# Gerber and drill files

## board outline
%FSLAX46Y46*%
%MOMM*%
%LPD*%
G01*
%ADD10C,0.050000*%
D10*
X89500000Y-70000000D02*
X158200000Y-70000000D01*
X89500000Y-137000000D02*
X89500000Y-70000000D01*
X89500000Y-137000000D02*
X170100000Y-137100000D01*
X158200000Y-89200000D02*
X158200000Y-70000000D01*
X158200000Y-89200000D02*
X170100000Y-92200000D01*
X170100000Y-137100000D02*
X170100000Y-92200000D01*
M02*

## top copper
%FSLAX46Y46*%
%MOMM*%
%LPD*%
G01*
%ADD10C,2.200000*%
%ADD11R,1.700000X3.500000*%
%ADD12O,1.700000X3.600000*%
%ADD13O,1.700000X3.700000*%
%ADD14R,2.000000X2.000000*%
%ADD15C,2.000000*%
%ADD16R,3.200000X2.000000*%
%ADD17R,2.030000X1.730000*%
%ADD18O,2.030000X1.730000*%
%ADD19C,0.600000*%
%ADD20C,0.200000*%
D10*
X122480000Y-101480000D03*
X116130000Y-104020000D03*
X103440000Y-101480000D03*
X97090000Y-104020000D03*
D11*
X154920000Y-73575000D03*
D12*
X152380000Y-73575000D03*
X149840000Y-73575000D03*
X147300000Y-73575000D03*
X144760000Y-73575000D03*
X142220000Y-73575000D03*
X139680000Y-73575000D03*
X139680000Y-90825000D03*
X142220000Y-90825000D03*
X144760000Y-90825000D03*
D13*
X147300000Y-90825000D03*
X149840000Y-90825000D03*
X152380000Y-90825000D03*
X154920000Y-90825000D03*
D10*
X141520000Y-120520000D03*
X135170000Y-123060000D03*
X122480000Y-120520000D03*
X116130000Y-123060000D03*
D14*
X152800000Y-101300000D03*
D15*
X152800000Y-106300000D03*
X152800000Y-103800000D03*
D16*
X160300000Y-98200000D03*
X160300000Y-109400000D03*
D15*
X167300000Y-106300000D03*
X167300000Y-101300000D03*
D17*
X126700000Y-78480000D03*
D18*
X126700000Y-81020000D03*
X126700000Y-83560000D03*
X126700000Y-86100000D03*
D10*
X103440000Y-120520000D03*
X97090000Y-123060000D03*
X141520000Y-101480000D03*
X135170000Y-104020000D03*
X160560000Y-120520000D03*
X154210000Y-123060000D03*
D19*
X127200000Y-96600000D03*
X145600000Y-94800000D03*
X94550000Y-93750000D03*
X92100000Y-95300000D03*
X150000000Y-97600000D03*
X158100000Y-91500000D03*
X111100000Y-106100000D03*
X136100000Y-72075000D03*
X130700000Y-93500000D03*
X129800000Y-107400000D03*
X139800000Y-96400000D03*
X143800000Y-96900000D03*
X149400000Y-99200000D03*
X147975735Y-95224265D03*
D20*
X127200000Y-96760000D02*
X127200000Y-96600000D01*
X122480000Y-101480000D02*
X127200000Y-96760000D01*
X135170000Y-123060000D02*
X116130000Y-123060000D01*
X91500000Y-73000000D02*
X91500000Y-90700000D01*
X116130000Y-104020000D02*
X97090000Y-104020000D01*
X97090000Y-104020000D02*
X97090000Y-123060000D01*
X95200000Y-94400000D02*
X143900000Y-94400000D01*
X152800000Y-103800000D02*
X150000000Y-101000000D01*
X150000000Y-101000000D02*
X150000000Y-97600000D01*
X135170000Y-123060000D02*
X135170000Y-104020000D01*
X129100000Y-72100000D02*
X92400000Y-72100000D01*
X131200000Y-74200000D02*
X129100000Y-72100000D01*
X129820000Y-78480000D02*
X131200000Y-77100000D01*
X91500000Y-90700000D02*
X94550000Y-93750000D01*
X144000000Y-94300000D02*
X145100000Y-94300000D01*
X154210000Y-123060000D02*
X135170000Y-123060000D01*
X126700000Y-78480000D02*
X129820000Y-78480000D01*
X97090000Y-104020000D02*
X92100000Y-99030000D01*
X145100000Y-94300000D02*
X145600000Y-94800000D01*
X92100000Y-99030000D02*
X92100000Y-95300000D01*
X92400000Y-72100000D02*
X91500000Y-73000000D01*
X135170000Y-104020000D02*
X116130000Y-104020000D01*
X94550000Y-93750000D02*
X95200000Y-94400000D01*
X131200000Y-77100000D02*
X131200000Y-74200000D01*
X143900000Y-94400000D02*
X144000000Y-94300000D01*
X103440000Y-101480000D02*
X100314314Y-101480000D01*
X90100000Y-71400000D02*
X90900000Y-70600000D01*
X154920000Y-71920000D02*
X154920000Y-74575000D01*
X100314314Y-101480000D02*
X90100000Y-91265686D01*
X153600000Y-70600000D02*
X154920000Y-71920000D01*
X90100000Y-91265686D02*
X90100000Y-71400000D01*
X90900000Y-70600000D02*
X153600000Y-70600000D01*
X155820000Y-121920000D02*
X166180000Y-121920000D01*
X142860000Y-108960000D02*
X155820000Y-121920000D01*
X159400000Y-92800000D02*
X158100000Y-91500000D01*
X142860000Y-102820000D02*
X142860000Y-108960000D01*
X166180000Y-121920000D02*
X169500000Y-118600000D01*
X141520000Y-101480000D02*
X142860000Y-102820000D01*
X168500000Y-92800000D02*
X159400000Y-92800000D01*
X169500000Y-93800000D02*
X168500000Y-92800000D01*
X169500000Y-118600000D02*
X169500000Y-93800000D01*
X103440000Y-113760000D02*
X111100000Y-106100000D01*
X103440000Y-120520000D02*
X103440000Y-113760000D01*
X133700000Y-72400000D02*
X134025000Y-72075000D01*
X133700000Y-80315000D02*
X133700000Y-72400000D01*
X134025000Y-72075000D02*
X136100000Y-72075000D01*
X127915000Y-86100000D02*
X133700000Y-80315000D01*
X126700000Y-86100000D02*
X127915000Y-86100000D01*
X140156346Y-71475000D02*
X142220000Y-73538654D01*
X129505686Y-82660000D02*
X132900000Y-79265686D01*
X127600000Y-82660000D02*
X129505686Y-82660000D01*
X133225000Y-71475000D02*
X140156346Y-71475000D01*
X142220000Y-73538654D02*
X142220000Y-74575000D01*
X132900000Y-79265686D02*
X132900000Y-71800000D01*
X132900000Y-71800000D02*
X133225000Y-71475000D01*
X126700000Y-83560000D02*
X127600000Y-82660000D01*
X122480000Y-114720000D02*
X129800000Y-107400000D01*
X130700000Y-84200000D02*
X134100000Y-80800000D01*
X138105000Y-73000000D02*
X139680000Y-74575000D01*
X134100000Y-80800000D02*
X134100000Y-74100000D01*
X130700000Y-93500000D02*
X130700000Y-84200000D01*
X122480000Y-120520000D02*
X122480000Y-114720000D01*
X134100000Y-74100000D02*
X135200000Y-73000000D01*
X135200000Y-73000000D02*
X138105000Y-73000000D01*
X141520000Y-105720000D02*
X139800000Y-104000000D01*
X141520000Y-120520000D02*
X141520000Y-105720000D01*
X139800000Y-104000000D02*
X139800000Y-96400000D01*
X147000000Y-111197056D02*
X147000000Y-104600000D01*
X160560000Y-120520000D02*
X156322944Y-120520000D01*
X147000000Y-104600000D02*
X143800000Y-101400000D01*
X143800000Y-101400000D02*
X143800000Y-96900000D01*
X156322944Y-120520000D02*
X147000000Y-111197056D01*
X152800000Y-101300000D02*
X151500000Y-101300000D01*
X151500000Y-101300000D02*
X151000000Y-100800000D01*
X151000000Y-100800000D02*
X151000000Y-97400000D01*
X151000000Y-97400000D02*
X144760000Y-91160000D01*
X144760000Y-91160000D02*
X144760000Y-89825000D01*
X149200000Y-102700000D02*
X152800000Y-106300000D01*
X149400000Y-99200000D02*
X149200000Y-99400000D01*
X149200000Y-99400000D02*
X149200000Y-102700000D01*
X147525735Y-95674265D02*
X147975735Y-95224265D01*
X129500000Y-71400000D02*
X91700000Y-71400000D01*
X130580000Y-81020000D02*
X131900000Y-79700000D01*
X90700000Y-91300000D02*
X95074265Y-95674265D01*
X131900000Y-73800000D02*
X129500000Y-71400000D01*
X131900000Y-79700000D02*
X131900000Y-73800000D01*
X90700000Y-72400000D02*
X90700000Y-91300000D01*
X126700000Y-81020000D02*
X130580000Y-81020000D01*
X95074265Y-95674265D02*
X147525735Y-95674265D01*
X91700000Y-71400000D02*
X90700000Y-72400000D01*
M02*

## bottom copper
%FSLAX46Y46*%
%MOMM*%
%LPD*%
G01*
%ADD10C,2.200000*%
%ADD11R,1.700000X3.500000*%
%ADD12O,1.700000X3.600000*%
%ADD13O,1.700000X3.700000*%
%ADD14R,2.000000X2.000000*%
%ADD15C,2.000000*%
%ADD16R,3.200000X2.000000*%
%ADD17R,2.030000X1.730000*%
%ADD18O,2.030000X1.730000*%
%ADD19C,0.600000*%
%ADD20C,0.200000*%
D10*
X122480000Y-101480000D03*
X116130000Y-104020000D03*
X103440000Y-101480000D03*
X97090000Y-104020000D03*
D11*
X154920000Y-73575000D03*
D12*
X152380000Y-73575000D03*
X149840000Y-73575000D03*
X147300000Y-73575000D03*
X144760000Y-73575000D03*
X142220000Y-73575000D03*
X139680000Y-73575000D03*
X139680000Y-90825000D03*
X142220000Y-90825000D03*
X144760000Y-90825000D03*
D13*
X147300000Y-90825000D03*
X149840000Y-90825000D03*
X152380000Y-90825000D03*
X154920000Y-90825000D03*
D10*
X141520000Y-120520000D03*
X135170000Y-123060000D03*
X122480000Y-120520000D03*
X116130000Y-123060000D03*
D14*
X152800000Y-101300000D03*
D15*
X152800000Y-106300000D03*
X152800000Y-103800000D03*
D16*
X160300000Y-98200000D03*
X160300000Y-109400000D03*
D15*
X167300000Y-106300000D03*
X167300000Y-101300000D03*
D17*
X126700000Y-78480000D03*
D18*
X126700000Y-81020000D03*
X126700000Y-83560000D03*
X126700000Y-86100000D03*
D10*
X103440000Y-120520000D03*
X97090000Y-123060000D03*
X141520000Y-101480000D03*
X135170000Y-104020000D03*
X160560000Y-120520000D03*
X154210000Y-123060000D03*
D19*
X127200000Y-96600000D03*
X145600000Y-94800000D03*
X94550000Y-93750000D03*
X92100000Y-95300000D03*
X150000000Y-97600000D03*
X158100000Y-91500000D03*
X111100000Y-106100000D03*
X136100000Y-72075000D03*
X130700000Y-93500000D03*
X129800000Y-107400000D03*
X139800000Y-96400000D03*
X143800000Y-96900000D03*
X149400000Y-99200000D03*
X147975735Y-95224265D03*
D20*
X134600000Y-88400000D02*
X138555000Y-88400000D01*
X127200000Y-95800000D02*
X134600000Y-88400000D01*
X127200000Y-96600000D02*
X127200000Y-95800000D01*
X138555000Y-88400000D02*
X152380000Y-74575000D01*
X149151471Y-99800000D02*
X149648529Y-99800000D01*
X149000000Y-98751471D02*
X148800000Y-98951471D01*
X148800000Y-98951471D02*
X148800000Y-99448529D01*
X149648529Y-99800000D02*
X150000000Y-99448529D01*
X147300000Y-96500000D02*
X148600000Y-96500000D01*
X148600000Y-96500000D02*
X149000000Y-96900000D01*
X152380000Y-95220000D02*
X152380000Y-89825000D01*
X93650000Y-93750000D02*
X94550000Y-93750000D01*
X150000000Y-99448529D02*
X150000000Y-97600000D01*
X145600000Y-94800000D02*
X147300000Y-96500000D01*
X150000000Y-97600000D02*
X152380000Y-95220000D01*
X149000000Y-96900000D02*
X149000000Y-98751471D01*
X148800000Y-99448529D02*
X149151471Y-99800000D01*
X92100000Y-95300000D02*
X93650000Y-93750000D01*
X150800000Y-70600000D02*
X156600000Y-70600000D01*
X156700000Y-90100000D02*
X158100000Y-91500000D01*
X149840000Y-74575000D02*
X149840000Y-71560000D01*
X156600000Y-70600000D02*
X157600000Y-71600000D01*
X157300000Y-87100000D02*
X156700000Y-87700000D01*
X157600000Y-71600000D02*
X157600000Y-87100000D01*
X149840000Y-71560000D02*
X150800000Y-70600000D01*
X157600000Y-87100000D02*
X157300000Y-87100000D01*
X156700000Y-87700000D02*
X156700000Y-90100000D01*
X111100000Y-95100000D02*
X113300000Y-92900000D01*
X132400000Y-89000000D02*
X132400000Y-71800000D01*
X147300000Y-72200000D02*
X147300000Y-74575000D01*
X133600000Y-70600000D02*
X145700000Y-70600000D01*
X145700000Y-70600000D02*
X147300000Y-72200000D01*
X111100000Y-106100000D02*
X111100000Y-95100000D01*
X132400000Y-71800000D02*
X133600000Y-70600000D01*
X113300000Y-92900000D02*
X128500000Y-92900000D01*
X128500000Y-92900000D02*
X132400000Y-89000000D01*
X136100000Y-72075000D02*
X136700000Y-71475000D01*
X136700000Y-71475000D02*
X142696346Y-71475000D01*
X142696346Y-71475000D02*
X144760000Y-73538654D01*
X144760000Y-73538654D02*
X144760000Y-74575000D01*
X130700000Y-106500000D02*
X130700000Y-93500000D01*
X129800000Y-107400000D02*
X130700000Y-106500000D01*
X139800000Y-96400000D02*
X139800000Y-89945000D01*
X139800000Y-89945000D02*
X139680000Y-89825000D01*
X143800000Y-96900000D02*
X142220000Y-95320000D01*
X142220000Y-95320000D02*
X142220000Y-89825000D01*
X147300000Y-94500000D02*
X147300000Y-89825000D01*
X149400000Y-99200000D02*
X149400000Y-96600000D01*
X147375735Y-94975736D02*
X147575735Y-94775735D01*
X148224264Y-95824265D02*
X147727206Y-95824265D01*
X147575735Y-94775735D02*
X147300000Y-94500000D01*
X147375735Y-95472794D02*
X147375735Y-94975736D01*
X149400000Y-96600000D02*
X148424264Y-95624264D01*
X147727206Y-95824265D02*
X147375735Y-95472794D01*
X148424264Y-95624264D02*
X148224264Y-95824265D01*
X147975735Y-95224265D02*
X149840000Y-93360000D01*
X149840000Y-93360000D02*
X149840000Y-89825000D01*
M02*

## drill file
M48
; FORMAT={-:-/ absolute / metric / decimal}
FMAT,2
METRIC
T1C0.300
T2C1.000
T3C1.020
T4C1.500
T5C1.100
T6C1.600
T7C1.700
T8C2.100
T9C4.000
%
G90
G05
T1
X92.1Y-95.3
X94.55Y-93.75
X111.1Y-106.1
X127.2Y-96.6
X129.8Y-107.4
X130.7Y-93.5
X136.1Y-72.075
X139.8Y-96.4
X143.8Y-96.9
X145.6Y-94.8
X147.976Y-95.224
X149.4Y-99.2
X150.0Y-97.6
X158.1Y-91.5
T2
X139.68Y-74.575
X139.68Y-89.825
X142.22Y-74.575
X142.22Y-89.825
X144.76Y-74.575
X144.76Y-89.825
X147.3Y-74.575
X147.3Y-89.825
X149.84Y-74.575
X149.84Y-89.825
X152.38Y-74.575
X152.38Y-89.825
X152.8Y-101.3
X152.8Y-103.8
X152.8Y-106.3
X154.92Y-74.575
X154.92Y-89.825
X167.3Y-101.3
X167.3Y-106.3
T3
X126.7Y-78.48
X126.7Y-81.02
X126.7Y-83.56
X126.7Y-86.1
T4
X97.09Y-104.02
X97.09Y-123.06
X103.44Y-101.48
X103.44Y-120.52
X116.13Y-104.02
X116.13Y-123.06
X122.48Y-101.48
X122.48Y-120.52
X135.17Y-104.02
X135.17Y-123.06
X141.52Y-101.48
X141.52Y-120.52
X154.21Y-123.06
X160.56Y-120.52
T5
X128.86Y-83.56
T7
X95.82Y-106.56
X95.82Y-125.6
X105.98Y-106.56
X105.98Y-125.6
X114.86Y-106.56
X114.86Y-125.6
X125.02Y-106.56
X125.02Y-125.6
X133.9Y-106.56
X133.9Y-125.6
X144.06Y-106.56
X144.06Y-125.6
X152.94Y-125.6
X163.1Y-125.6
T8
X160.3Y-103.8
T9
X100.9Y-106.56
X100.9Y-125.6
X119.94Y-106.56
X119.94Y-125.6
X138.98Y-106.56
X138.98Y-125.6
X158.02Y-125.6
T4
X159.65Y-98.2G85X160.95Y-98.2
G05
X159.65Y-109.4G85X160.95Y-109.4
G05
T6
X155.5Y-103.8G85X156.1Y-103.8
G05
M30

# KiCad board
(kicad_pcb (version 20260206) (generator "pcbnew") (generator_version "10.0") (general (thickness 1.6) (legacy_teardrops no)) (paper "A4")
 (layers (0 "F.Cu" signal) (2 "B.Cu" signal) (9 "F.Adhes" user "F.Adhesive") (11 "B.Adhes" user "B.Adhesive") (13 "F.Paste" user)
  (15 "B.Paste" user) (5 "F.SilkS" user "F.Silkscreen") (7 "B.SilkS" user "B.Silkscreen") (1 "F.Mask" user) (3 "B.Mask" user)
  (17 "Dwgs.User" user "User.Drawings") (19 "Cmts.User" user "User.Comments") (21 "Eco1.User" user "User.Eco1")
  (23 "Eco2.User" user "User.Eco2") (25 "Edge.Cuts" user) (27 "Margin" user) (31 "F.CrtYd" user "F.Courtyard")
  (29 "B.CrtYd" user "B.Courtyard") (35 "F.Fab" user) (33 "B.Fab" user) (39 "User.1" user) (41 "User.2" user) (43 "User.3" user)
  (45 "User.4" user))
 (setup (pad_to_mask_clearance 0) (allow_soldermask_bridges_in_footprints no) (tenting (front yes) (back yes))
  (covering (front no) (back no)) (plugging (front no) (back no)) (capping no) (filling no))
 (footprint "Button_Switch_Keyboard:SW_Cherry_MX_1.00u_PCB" (layer "F.Cu") (at 122.48 101.48)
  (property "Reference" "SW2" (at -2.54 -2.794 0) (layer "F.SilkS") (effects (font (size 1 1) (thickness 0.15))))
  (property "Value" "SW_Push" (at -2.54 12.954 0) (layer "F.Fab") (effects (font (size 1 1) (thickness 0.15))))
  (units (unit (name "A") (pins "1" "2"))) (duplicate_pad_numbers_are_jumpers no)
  (pad "" np_thru_hole circle (at -7.62 5.08) (size 1.7 1.7) (drill 1.7) (layers "*.Cu" "*.Mask"))
  (pad "" np_thru_hole circle (at -2.54 5.08) (size 4 4) (drill 4) (layers "*.Cu" "*.Mask"))
  (pad "" np_thru_hole circle (at 2.54 5.08) (size 1.7 1.7) (drill 1.7) (layers "*.Cu" "*.Mask"))
  (pad "1" thru_hole circle (at 0 0) (size 2.2 2.2) (drill 1.5) (layers "*.Cu" "*.Mask") (remove_unused_layers no) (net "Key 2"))
  (pad "2" thru_hole circle (at -6.35 2.54) (size 2.2 2.2) (drill 1.5) (layers "*.Cu" "*.Mask") (remove_unused_layers no) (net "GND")))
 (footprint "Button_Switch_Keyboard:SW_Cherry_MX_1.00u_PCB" (layer "F.Cu") (at 103.44 101.48)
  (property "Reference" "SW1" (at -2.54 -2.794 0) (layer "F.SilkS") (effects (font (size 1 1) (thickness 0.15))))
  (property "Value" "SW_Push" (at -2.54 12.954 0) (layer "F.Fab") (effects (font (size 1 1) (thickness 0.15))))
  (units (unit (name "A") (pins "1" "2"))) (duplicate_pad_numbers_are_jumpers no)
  (pad "" np_thru_hole circle (at -7.62 5.08) (size 1.7 1.7) (drill 1.7) (layers "*.Cu" "*.Mask"))
  (pad "" np_thru_hole circle (at -2.54 5.08) (size 4 4) (drill 4) (layers "*.Cu" "*.Mask"))
  (pad "" np_thru_hole circle (at 2.54 5.08) (size 1.7 1.7) (drill 1.7) (layers "*.Cu" "*.Mask"))
  (pad "1" thru_hole circle (at 0 0) (size 2.2 2.2) (drill 1.5) (layers "*.Cu" "*.Mask") (remove_unused_layers no) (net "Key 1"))
  (pad "2" thru_hole circle (at -6.35 2.54) (size 2.2 2.2) (drill 1.5) (layers "*.Cu" "*.Mask") (remove_unused_layers no) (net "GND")))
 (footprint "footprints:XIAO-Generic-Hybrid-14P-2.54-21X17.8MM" (layer "F.Cu") (at 147.3 82.2 -90)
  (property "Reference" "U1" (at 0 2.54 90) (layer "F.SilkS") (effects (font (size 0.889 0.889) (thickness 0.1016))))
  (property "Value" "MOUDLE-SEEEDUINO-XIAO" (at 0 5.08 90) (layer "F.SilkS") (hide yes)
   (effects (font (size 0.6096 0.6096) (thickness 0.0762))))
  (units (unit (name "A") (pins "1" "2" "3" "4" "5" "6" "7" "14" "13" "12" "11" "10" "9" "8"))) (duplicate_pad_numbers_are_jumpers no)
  (pad "1" thru_hole rect (at -7.625 -7.62 270) (size 3.5 1.7) (drill 1 (offset -1 0)) (layers "*.Cu" "*.Mask") (remove_unused_layers no)
   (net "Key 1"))
  (pad "2" thru_hole oval (at -7.625 -5.08 270) (size 3.6 1.7) (drill 1 (offset -1 0)) (layers "*.Cu" "*.Mask") (remove_unused_layers no)
   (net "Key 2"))
  (pad "3" thru_hole oval (at -7.625 -2.54 270) (size 3.6 1.7) (drill 1 (offset -1 0)) (layers "*.Cu" "*.Mask") (remove_unused_layers no)
   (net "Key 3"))
  (pad "4" thru_hole oval (at -7.625 0 270) (size 3.6 1.7) (drill 1 (offset -1 0)) (layers "*.Cu" "*.Mask") (remove_unused_layers no)
   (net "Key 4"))
  (pad "5" thru_hole oval (at -7.625 2.54 270) (size 3.6 1.7) (drill 1 (offset -1 0)) (layers "*.Cu" "*.Mask") (remove_unused_layers no)
   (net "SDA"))
  (pad "6" thru_hole oval (at -7.625 5.08 90) (size 3.6 1.7) (drill 1 (offset 1 0)) (layers "*.Cu" "*.Mask") (remove_unused_layers no)
   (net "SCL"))
  (pad "7" thru_hole oval (at -7.625 7.62 270) (size 3.6 1.7) (drill 1 (offset -1 0)) (layers "*.Cu" "*.Mask") (remove_unused_layers no)
   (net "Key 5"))
  (pad "8" thru_hole oval (at 7.625 7.62 270) (size 3.6 1.7) (drill 1 (offset 1 0)) (layers "*.Cu" "*.Mask") (remove_unused_layers no)
   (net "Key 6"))
  (pad "9" thru_hole oval (at 7.625 5.08 270) (size 3.6 1.7) (drill 1 (offset 1 0)) (layers "*.Cu" "*.Mask") (remove_unused_layers no)
   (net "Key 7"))
  (pad "10" thru_hole oval (at 7.625 2.54 270) (size 3.6 1.7) (drill 1 (offset 1 0)) (layers "*.Cu" "*.Mask") (remove_unused_layers no)
   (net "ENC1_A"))
  (pad "11" thru_hole oval (at 7.625 0 270) (size 3.7 1.7) (drill 1 (offset 1 0)) (layers "*.Cu" "*.Mask") (remove_unused_layers no)
   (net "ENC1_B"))
  (pad "12" thru_hole oval (at 7.625 -2.54 270) (size 3.7 1.7) (drill 1 (offset 1 0)) (layers "*.Cu" "*.Mask") (remove_unused_layers no)
   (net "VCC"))
  (pad "13" thru_hole oval (at 7.625 -5.08 270) (size 3.7 1.7) (drill 1 (offset 1 0)) (layers "*.Cu" "*.Mask") (remove_unused_layers no)
   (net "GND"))
  (pad "14" thru_hole oval (at 7.625 -7.62 270) (size 3.7 1.7) (drill 1 (offset 1 0)) (layers "*.Cu" "*.Mask") (remove_unused_layers no)
   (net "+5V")))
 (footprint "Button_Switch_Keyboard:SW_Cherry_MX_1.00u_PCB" (layer "F.Cu") (at 141.52 120.52)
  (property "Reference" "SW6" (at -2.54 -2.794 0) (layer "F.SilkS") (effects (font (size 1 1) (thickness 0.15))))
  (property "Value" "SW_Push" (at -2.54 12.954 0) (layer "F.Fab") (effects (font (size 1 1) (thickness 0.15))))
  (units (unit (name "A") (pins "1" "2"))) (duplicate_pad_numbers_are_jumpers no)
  (pad "" np_thru_hole circle (at -7.62 5.08) (size 1.7 1.7) (drill 1.7) (layers "*.Cu" "*.Mask"))
  (pad "" np_thru_hole circle (at -2.54 5.08) (size 4 4) (drill 4) (layers "*.Cu" "*.Mask"))
  (pad "" np_thru_hole circle (at 2.54 5.08) (size 1.7 1.7) (drill 1.7) (layers "*.Cu" "*.Mask"))
  (pad "1" thru_hole circle (at 0 0) (size 2.2 2.2) (drill 1.5) (layers "*.Cu" "*.Mask") (remove_unused_layers no) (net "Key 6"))
  (pad "2" thru_hole circle (at -6.35 2.54) (size 2.2 2.2) (drill 1.5) (layers "*.Cu" "*.Mask") (remove_unused_layers no) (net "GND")))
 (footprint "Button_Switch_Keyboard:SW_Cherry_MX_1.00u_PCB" (layer "F.Cu") (at 122.48 120.52)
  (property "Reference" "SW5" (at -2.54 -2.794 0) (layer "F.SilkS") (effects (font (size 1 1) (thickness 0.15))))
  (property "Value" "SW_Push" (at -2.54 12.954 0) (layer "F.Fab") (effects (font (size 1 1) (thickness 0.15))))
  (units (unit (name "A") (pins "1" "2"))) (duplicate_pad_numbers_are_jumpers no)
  (pad "" np_thru_hole circle (at -7.62 5.08) (size 1.7 1.7) (drill 1.7) (layers "*.Cu" "*.Mask"))
  (pad "" np_thru_hole circle (at -2.54 5.08) (size 4 4) (drill 4) (layers "*.Cu" "*.Mask"))
  (pad "" np_thru_hole circle (at 2.54 5.08) (size 1.7 1.7) (drill 1.7) (layers "*.Cu" "*.Mask"))
  (pad "1" thru_hole circle (at 0 0) (size 2.2 2.2) (drill 1.5) (layers "*.Cu" "*.Mask") (remove_unused_layers no) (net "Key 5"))
  (pad "2" thru_hole circle (at -6.35 2.54) (size 2.2 2.2) (drill 1.5) (layers "*.Cu" "*.Mask") (remove_unused_layers no) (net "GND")))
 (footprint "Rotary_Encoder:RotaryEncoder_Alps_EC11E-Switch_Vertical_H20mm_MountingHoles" (layer "F.Cu") (at 152.8 101.3)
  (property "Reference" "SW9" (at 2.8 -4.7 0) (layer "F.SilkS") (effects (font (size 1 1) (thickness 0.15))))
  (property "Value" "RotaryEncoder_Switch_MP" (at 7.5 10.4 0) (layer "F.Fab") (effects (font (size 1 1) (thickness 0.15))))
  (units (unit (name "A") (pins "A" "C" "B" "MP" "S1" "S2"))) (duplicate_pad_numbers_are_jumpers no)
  (pad "" np_thru_hole oval (at 3 2.5) (size 2.2 1.6) (drill oval 2.2 1.6) (layers "*.Mask"))
  (pad "" np_thru_hole circle (at 7.5 2.5) (size 2.1 2.1) (drill 2.1) (layers "*.Mask"))
  (pad "A" thru_hole rect (at 0 0) (size 2 2) (drill 1) (layers "*.Cu" "*.Mask") (remove_unused_layers no) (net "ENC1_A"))
  (pad "B" thru_hole circle (at 0 5) (size 2 2) (drill 1) (layers "*.Cu" "*.Mask") (remove_unused_layers no) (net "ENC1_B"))
  (pad "C" thru_hole circle (at 0 2.5) (size 2 2) (drill 1) (layers "*.Cu" "*.Mask") (remove_unused_layers no) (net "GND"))
  (pad "MP" thru_hole rect (at 7.5 -3.1) (size 3.2 2) (drill oval 2.8 1.5) (layers "*.Cu" "*.Mask") (remove_unused_layers no)
   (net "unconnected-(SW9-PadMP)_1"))
  (pad "MP" thru_hole rect (at 7.5 8.1) (size 3.2 2) (drill oval 2.8 1.5) (layers "*.Cu" "*.Mask") (remove_unused_layers no)
   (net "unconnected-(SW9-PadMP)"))
  (pad "S1" thru_hole circle (at 14.5 5) (size 2 2) (drill 1) (layers "*.Cu" "*.Mask") (remove_unused_layers no)
   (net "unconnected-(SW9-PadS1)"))
  (pad "S2" thru_hole circle (at 14.5 0) (size 2 2) (drill 1) (layers "*.Cu" "*.Mask") (remove_unused_layers no)
   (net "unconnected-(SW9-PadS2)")))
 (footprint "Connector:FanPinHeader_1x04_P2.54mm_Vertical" (layer "F.Cu") (at 126.7 78.48 -90)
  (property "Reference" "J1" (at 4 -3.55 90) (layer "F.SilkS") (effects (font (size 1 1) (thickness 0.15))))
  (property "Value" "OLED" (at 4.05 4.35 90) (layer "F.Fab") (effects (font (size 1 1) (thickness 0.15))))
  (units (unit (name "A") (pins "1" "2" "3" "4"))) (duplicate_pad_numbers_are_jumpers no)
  (pad "" np_thru_hole circle (at 5.08 -2.16) (size 1.1 1.1) (drill 1.1) (layers "*.Cu" "*.Mask"))
  (pad "1" thru_hole rect (at 0 0) (size 2.03 1.73) (drill 1.02) (layers "*.Cu" "*.Mask") (remove_unused_layers no) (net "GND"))
  (pad "2" thru_hole oval (at 2.54 0) (size 2.03 1.73) (drill 1.02) (layers "*.Cu" "*.Mask") (remove_unused_layers no) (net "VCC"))
  (pad "3" thru_hole oval (at 5.08 0) (size 2.03 1.73) (drill 1.02) (layers "*.Cu" "*.Mask") (remove_unused_layers no) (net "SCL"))
  (pad "4" thru_hole oval (at 7.62 0) (size 2.03 1.73) (drill 1.02) (layers "*.Cu" "*.Mask") (remove_unused_layers no) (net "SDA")))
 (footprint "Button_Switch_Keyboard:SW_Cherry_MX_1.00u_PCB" (layer "F.Cu") (at 103.44 120.52)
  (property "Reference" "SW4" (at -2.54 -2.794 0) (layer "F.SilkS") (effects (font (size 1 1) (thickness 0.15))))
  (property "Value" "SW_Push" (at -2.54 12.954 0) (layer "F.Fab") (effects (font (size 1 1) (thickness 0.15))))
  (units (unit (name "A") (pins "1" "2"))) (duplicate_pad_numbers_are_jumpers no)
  (pad "" np_thru_hole circle (at -7.62 5.08) (size 1.7 1.7) (drill 1.7) (layers "*.Cu" "*.Mask"))
  (pad "" np_thru_hole circle (at -2.54 5.08) (size 4 4) (drill 4) (layers "*.Cu" "*.Mask"))
  (pad "" np_thru_hole circle (at 2.54 5.08) (size 1.7 1.7) (drill 1.7) (layers "*.Cu" "*.Mask"))
  (pad "1" thru_hole circle (at 0 0) (size 2.2 2.2) (drill 1.5) (layers "*.Cu" "*.Mask") (remove_unused_layers no) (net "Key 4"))
  (pad "2" thru_hole circle (at -6.35 2.54) (size 2.2 2.2) (drill 1.5) (layers "*.Cu" "*.Mask") (remove_unused_layers no) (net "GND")))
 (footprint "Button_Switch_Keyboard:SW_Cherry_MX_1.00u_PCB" (layer "F.Cu") (at 141.52 101.48)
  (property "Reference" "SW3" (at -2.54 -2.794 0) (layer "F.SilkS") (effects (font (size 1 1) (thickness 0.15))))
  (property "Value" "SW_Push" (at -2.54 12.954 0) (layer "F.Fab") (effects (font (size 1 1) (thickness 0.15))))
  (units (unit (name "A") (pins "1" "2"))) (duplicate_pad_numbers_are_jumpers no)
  (pad "" np_thru_hole circle (at -7.62 5.08) (size 1.7 1.7) (drill 1.7) (layers "*.Cu" "*.Mask"))
  (pad "" np_thru_hole circle (at -2.54 5.08) (size 4 4) (drill 4) (layers "*.Cu" "*.Mask"))
  (pad "" np_thru_hole circle (at 2.54 5.08) (size 1.7 1.7) (drill 1.7) (layers "*.Cu" "*.Mask"))
  (pad "1" thru_hole circle (at 0 0) (size 2.2 2.2) (drill 1.5) (layers "*.Cu" "*.Mask") (remove_unused_layers no) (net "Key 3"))
  (pad "2" thru_hole circle (at -6.35 2.54) (size 2.2 2.2) (drill 1.5) (layers "*.Cu" "*.Mask") (remove_unused_layers no) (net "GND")))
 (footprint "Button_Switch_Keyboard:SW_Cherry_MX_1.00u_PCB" (layer "F.Cu") (at 160.56 120.52)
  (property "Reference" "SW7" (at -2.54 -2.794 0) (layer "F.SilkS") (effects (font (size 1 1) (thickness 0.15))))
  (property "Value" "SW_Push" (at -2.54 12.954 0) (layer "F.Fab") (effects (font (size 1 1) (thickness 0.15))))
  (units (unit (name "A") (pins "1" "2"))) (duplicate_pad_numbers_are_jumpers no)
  (pad "" np_thru_hole circle (at -7.62 5.08) (size 1.7 1.7) (drill 1.7) (layers "*.Cu" "*.Mask"))
  (pad "" np_thru_hole circle (at -2.54 5.08) (size 4 4) (drill 4) (layers "*.Cu" "*.Mask"))
  (pad "" np_thru_hole circle (at 2.54 5.08) (size 1.7 1.7) (drill 1.7) (layers "*.Cu" "*.Mask"))
  (pad "1" thru_hole circle (at 0 0) (size 2.2 2.2) (drill 1.5) (layers "*.Cu" "*.Mask") (remove_unused_layers no) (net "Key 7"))
  (pad "2" thru_hole circle (at -6.35 2.54) (size 2.2 2.2) (drill 1.5) (layers "*.Cu" "*.Mask") (remove_unused_layers no) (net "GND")))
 (gr_line (start 89.5 70) (end 158.2 70) (stroke (width 0.05) (type default)) (layer "Edge.Cuts"))
 (gr_line (start 89.5 137) (end 89.5 70) (stroke (width 0.05) (type default)) (layer "Edge.Cuts"))
 (gr_line (start 89.5 137) (end 170.1 137.1) (stroke (width 0.05) (type default)) (layer "Edge.Cuts"))
 (gr_line (start 158.2 89.2) (end 158.2 70) (stroke (width 0.05) (type default)) (layer "Edge.Cuts"))
 (gr_line (start 158.2 89.2) (end 170.1 92.2) (stroke (width 0.05) (type default)) (layer "Edge.Cuts"))
 (gr_line (start 170.1 137.1) (end 170.1 92.2) (stroke (width 0.05) (type default)) (layer "Edge.Cuts"))
 (segment (start 127.2 96.76) (end 127.2 96.6) (width 0.2) (layer "F.Cu") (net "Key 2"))
 (segment (start 122.48 101.48) (end 127.2 96.76) (width 0.2) (layer "F.Cu") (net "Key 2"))
 (via (at 127.2 96.6) (size 0.6) (drill 0.3) (layers "F.Cu" "B.Cu") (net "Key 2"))
 (segment (start 134.6 88.4) (end 138.555 88.4) (width 0.2) (layer "B.Cu") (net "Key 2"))
 (segment (start 127.2 95.8) (end 134.6 88.4) (width 0.2) (layer "B.Cu") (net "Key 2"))
 (segment (start 127.2 96.6) (end 127.2 95.8) (width 0.2) (layer "B.Cu") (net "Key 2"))
 (segment (start 138.555 88.4) (end 152.38 74.575) (width 0.2) (layer "B.Cu") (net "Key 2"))
 (segment (start 135.17 123.06) (end 116.13 123.06) (width 0.2) (layer "F.Cu") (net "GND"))
 (segment (start 91.5 73) (end 91.5 90.7) (width 0.2) (layer "F.Cu") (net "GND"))
 (segment (start 116.13 104.02) (end 97.09 104.02) (width 0.2) (layer "F.Cu") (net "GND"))
 (segment (start 97.09 104.02) (end 97.09 123.06) (width 0.2) (layer "F.Cu") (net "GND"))
 (segment (start 95.2 94.4) (end 143.9 94.4) (width 0.2) (layer "F.Cu") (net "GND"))
 (segment (start 152.8 103.8) (end 150 101) (width 0.2) (layer "F.Cu") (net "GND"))
 (segment (start 150 101) (end 150 97.6) (width 0.2) (layer "F.Cu") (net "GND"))
 (segment (start 135.17 123.06) (end 135.17 104.02) (width 0.2) (layer "F.Cu") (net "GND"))
 (segment (start 129.1 72.1) (end 92.4 72.1) (width 0.2) (layer "F.Cu") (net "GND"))
 (segment (start 131.2 74.2) (end 129.1 72.1) (width 0.2) (layer "F.Cu") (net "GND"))
 (segment (start 129.82 78.48) (end 131.2 77.1) (width 0.2) (layer "F.Cu") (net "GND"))
 (segment (start 91.5 90.7) (end 94.55 93.75) (width 0.2) (layer "F.Cu") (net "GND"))
 (segment (start 144 94.3) (end 145.1 94.3) (width 0.2) (layer "F.Cu") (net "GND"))
 (segment (start 154.21 123.06) (end 135.17 123.06) (width 0.2) (layer "F.Cu") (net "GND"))
 (segment (start 126.7 78.48) (end 129.82 78.48) (width 0.2) (layer "F.Cu") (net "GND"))
 (segment (start 97.09 104.02) (end 92.1 99.03) (width 0.2) (layer "F.Cu") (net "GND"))
 (segment (start 145.1 94.3) (end 145.6 94.8) (width 0.2) (layer "F.Cu") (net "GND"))
 (segment (start 92.1 99.03) (end 92.1 95.3) (width 0.2) (layer "F.Cu") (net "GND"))
 (segment (start 92.4 72.1) (end 91.5 73) (width 0.2) (layer "F.Cu") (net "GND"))
 (segment (start 135.17 104.02) (end 116.13 104.02) (width 0.2) (layer "F.Cu") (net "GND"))
 (segment (start 94.55 93.75) (end 95.2 94.4) (width 0.2) (layer "F.Cu") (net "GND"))
 (segment (start 131.2 77.1) (end 131.2 74.2) (width 0.2) (layer "F.Cu") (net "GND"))
 (segment (start 143.9 94.4) (end 144 94.3) (width 0.2) (layer "F.Cu") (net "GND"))
 (via (at 145.6 94.8) (size 0.6) (drill 0.3) (layers "F.Cu" "B.Cu") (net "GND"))
 (via (at 94.55 93.75) (size 0.6) (drill 0.3) (layers "F.Cu" "B.Cu") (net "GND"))
 (via (at 92.1 95.3) (size 0.6) (drill 0.3) (layers "F.Cu" "B.Cu") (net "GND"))
 (via (at 150 97.6) (size 0.6) (drill 0.3) (layers "F.Cu" "B.Cu") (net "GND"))
 (segment (start 149.151471 99.8) (end 149.648529 99.8) (width 0.2) (layer "B.Cu") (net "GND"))
 (segment (start 149 98.751471) (end 148.8 98.951471) (width 0.2) (layer "B.Cu") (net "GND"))
 (segment (start 148.8 98.951471) (end 148.8 99.448529) (width 0.2) (layer "B.Cu") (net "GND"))
 (segment (start 149.648529 99.8) (end 150 99.448529) (width 0.2) (layer "B.Cu") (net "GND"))
 (segment (start 147.3 96.5) (end 148.6 96.5) (width 0.2) (layer "B.Cu") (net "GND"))
 (segment (start 148.6 96.5) (end 149 96.9) (width 0.2) (layer "B.Cu") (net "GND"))
 (segment (start 152.38 95.22) (end 152.38 89.825) (width 0.2) (layer "B.Cu") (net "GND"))
 (segment (start 93.65 93.75) (end 94.55 93.75) (width 0.2) (layer "B.Cu") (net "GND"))
 (segment (start 150 99.448529) (end 150 97.6) (width 0.2) (layer "B.Cu") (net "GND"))
 (segment (start 145.6 94.8) (end 147.3 96.5) (width 0.2) (layer "B.Cu") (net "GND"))
 (segment (start 150 97.6) (end 152.38 95.22) (width 0.2) (layer "B.Cu") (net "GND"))
 (segment (start 149 96.9) (end 149 98.751471) (width 0.2) (layer "B.Cu") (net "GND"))
 (segment (start 148.8 99.448529) (end 149.151471 99.8) (width 0.2) (layer "B.Cu") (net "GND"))
 (segment (start 92.1 95.3) (end 93.65 93.75) (width 0.2) (layer "B.Cu") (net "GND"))
 (segment (start 103.44 101.48) (end 100.314314 101.48) (width 0.2) (layer "F.Cu") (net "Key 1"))
 (segment (start 90.1 71.4) (end 90.9 70.6) (width 0.2) (layer "F.Cu") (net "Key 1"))
 (segment (start 154.92 71.92) (end 154.92 74.575) (width 0.2) (layer "F.Cu") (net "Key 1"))
 (segment (start 100.314314 101.48) (end 90.1 91.265686) (width 0.2) (layer "F.Cu") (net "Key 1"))
 (segment (start 153.6 70.6) (end 154.92 71.92) (width 0.2) (layer "F.Cu") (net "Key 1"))
 (segment (start 90.1 91.265686) (end 90.1 71.4) (width 0.2) (layer "F.Cu") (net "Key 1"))
 (segment (start 90.9 70.6) (end 153.6 70.6) (width 0.2) (layer "F.Cu") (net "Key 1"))
 (segment (start 155.82 121.92) (end 166.18 121.92) (width 0.2) (layer "F.Cu") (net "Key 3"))
 (segment (start 142.86 108.96) (end 155.82 121.92) (width 0.2) (layer "F.Cu") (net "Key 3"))
 (segment (start 159.4 92.8) (end 158.1 91.5) (width 0.2) (layer "F.Cu") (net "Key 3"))
 (segment (start 142.86 102.82) (end 142.86 108.96) (width 0.2) (layer "F.Cu") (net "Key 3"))
 (segment (start 166.18 121.92) (end 169.5 118.6) (width 0.2) (layer "F.Cu") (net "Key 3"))
 (segment (start 141.52 101.48) (end 142.86 102.82) (width 0.2) (layer "F.Cu") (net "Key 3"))
 (segment (start 168.5 92.8) (end 159.4 92.8) (width 0.2) (layer "F.Cu") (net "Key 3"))
 (segment (start 169.5 93.8) (end 168.5 92.8) (width 0.2) (layer "F.Cu") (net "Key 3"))
 (segment (start 169.5 118.6) (end 169.5 93.8) (width 0.2) (layer "F.Cu") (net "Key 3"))
 (via (at 158.1 91.5) (size 0.6) (drill 0.3) (layers "F.Cu" "B.Cu") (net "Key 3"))
 (segment (start 150.8 70.6) (end 156.6 70.6) (width 0.2) (layer "B.Cu") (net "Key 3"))
 (segment (start 156.7 90.1) (end 158.1 91.5) (width 0.2) (layer "B.Cu") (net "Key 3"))
 (segment (start 149.84 74.575) (end 149.84 71.56) (width 0.2) (layer "B.Cu") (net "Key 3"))
 (segment (start 156.6 70.6) (end 157.6 71.6) (width 0.2) (layer "B.Cu") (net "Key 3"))
 (segment (start 157.3 87.1) (end 156.7 87.7) (width 0.2) (layer "B.Cu") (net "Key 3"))
 (segment (start 157.6 71.6) (end 157.6 87.1) (width 0.2) (layer "B.Cu") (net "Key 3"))
 (segment (start 149.84 71.56) (end 150.8 70.6) (width 0.2) (layer "B.Cu") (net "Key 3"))
 (segment (start 157.6 87.1) (end 157.3 87.1) (width 0.2) (layer "B.Cu") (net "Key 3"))
 (segment (start 156.7 87.7) (end 156.7 90.1) (width 0.2) (layer "B.Cu") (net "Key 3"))
 (segment (start 103.44 113.76) (end 111.1 106.1) (width 0.2) (layer "F.Cu") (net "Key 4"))
 (segment (start 103.44 120.52) (end 103.44 113.76) (width 0.2) (layer "F.Cu") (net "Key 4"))
 (via (at 111.1 106.1) (size 0.6) (drill 0.3) (layers "F.Cu" "B.Cu") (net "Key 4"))
 (segment (start 111.1 95.1) (end 113.3 92.9) (width 0.2) (layer "B.Cu") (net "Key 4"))
 (segment (start 132.4 89) (end 132.4 71.8) (width 0.2) (layer "B.Cu") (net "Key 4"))
 (segment (start 147.3 72.2) (end 147.3 74.575) (width 0.2) (layer "B.Cu") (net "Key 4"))
 (segment (start 133.6 70.6) (end 145.7 70.6) (width 0.2) (layer "B.Cu") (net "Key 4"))
 (segment (start 145.7 70.6) (end 147.3 72.2) (width 0.2) (layer "B.Cu") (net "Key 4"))
 (segment (start 111.1 106.1) (end 111.1 95.1) (width 0.2) (layer "B.Cu") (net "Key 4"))
 (segment (start 132.4 71.8) (end 133.6 70.6) (width 0.2) (layer "B.Cu") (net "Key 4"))
 (segment (start 113.3 92.9) (end 128.5 92.9) (width 0.2) (layer "B.Cu") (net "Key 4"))
 (segment (start 128.5 92.9) (end 132.4 89) (width 0.2) (layer "B.Cu") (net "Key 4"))
 (segment (start 133.7 72.4) (end 134.025 72.075) (width 0.2) (layer "F.Cu") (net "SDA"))
 (segment (start 133.7 80.315) (end 133.7 72.4) (width 0.2) (layer "F.Cu") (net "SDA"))
 (segment (start 134.025 72.075) (end 136.1 72.075) (width 0.2) (layer "F.Cu") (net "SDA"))
 (segment (start 127.915 86.1) (end 133.7 80.315) (width 0.2) (layer "F.Cu") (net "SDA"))
 (segment (start 126.7 86.1) (end 127.915 86.1) (width 0.2) (layer "F.Cu") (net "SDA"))
 (via (at 136.1 72.075) (size 0.6) (drill 0.3) (layers "F.Cu" "B.Cu") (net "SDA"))
 (segment (start 136.1 72.075) (end 136.7 71.475) (width 0.2) (layer "B.Cu") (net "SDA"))
 (segment (start 136.7 71.475) (end 142.696346 71.475) (width 0.2) (layer "B.Cu") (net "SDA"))
 (segment (start 142.696346 71.475) (end 144.76 73.538654) (width 0.2) (layer "B.Cu") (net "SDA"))
 (segment (start 144.76 73.538654) (end 144.76 74.575) (width 0.2) (layer "B.Cu") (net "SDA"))
 (segment (start 140.156346 71.475) (end 142.22 73.538654) (width 0.2) (layer "F.Cu") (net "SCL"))
 (segment (start 129.505686 82.66) (end 132.9 79.265686) (width 0.2) (layer "F.Cu") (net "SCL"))
 (segment (start 127.6 82.66) (end 129.505686 82.66) (width 0.2) (layer "F.Cu") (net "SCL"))
 (segment (start 133.225 71.475) (end 140.156346 71.475) (width 0.2) (layer "F.Cu") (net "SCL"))
 (segment (start 142.22 73.538654) (end 142.22 74.575) (width 0.2) (layer "F.Cu") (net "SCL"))
 (segment (start 132.9 79.265686) (end 132.9 71.8) (width 0.2) (layer "F.Cu") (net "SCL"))
 (segment (start 132.9 71.8) (end 133.225 71.475) (width 0.2) (layer "F.Cu") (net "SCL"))
 (segment (start 126.7 83.56) (end 127.6 82.66) (width 0.2) (layer "F.Cu") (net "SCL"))
 (segment (start 122.48 114.72) (end 129.8 107.4) (width 0.2) (layer "F.Cu") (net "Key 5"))
 (segment (start 130.7 84.2) (end 134.1 80.8) (width 0.2) (layer "F.Cu") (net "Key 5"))
 (segment (start 138.105 73) (end 139.68 74.575) (width 0.2) (layer "F.Cu") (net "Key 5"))
 (segment (start 134.1 80.8) (end 134.1 74.1) (width 0.2) (layer "F.Cu") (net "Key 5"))
 (segment (start 130.7 93.5) (end 130.7 84.2) (width 0.2) (layer "F.Cu") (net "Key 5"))
 (segment (start 122.48 120.52) (end 122.48 114.72) (width 0.2) (layer "F.Cu") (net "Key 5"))
 (segment (start 134.1 74.1) (end 135.2 73) (width 0.2) (layer "F.Cu") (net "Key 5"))
 (segment (start 135.2 73) (end 138.105 73) (width 0.2) (layer "F.Cu") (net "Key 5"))
 (via (at 130.7 93.5) (size 0.6) (drill 0.3) (layers "F.Cu" "B.Cu") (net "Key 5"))
 (via (at 129.8 107.4) (size 0.6) (drill 0.3) (layers "F.Cu" "B.Cu") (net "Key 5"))
 (segment (start 130.7 106.5) (end 130.7 93.5) (width 0.2) (layer "B.Cu") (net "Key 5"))
 (segment (start 129.8 107.4) (end 130.7 106.5) (width 0.2) (layer "B.Cu") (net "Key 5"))
 (segment (start 141.52 105.72) (end 139.8 104) (width 0.2) (layer "F.Cu") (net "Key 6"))
 (segment (start 141.52 120.52) (end 141.52 105.72) (width 0.2) (layer "F.Cu") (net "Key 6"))
 (segment (start 139.8 104) (end 139.8 96.4) (width 0.2) (layer "F.Cu") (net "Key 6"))
 (via (at 139.8 96.4) (size 0.6) (drill 0.3) (layers "F.Cu" "B.Cu") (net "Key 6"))
 (segment (start 139.8 96.4) (end 139.8 89.945) (width 0.2) (layer "B.Cu") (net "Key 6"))
 (segment (start 139.8 89.945) (end 139.68 89.825) (width 0.2) (layer "B.Cu") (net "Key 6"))
 (segment (start 147 111.197056) (end 147 104.6) (width 0.2) (layer "F.Cu") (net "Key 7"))
 (segment (start 160.56 120.52) (end 156.322944 120.52) (width 0.2) (layer "F.Cu") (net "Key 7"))
 (segment (start 147 104.6) (end 143.8 101.4) (width 0.2) (layer "F.Cu") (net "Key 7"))
 (segment (start 143.8 101.4) (end 143.8 96.9) (width 0.2) (layer "F.Cu") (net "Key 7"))
 (segment (start 156.322944 120.52) (end 147 111.197056) (width 0.2) (layer "F.Cu") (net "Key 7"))
 (via (at 143.8 96.9) (size 0.6) (drill 0.3) (layers "F.Cu" "B.Cu") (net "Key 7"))
 (segment (start 143.8 96.9) (end 142.22 95.32) (width 0.2) (layer "B.Cu") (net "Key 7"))
 (segment (start 142.22 95.32) (end 142.22 89.825) (width 0.2) (layer "B.Cu") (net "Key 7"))
 (segment (start 152.8 101.3) (end 151.5 101.3) (width 0.2) (layer "F.Cu") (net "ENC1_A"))
 (segment (start 151.5 101.3) (end 151 100.8) (width 0.2) (layer "F.Cu") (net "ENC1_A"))
 (segment (start 151 100.8) (end 151 97.4) (width 0.2) (layer "F.Cu") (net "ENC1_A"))
 (segment (start 151 97.4) (end 144.76 91.16) (width 0.2) (layer "F.Cu") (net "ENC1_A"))
 (segment (start 144.76 91.16) (end 144.76 89.825) (width 0.2) (layer "F.Cu") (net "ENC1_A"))
 (segment (start 149.2 102.7) (end 152.8 106.3) (width 0.2) (layer "F.Cu") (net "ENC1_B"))
 (segment (start 149.4 99.2) (end 149.2 99.4) (width 0.2) (layer "F.Cu") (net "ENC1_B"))
 (segment (start 149.2 99.4) (end 149.2 102.7) (width 0.2) (layer "F.Cu") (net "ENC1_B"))
 (via (at 149.4 99.2) (size 0.6) (drill 0.3) (layers "F.Cu" "B.Cu") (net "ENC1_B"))
 (segment (start 147.3 94.5) (end 147.3 89.825) (width 0.2) (layer "B.Cu") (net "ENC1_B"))
 (segment (start 149.4 99.2) (end 149.4 96.6) (width 0.2) (layer "B.Cu") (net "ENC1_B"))
 (segment (start 147.375735 94.975736) (end 147.575735 94.775735) (width 0.2) (layer "B.Cu") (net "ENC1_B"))
 (segment (start 148.224264 95.824265) (end 147.727206 95.824265) (width 0.2) (layer "B.Cu") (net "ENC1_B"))
 (segment (start 147.575735 94.775735) (end 147.3 94.5) (width 0.2) (layer "B.Cu") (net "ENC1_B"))
 (segment (start 147.375735 95.472794) (end 147.375735 94.975736) (width 0.2) (layer "B.Cu") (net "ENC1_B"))
 (segment (start 149.4 96.6) (end 148.424264 95.624264) (width 0.2) (layer "B.Cu") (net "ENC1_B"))
 (segment (start 147.727206 95.824265) (end 147.375735 95.472794) (width 0.2) (layer "B.Cu") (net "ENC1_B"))
 (segment (start 148.424264 95.624264) (end 148.224264 95.824265) (width 0.2) (layer "B.Cu") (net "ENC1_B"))
 (segment (start 147.525735 95.674265) (end 147.975735 95.224265) (width 0.2) (layer "F.Cu") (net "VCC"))
 (segment (start 129.5 71.4) (end 91.7 71.4) (width 0.2) (layer "F.Cu") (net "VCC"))
 (segment (start 130.58 81.02) (end 131.9 79.7) (width 0.2) (layer "F.Cu") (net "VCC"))
 (segment (start 90.7 91.3) (end 95.074265 95.674265) (width 0.2) (layer "F.Cu") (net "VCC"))
 (segment (start 131.9 73.8) (end 129.5 71.4) (width 0.2) (layer "F.Cu") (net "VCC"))
 (segment (start 131.9 79.7) (end 131.9 73.8) (width 0.2) (layer "F.Cu") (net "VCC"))
 (segment (start 90.7 72.4) (end 90.7 91.3) (width 0.2) (layer "F.Cu") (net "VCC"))
 (segment (start 126.7 81.02) (end 130.58 81.02) (width 0.2) (layer "F.Cu") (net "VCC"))
 (segment (start 95.074265 95.674265) (end 147.525735 95.674265) (width 0.2) (layer "F.Cu") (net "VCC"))
 (segment (start 91.7 71.4) (end 90.7 72.4) (width 0.2) (layer "F.Cu") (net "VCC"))
 (via (at 147.975735 95.224265) (size 0.6) (drill 0.3) (layers "F.Cu" "B.Cu") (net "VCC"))
 (segment (start 147.975735 95.224265) (end 149.84 93.36) (width 0.2) (layer "B.Cu") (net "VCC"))
 (segment (start 149.84 93.36) (end 149.84 89.825) (width 0.2) (layer "B.Cu") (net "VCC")))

